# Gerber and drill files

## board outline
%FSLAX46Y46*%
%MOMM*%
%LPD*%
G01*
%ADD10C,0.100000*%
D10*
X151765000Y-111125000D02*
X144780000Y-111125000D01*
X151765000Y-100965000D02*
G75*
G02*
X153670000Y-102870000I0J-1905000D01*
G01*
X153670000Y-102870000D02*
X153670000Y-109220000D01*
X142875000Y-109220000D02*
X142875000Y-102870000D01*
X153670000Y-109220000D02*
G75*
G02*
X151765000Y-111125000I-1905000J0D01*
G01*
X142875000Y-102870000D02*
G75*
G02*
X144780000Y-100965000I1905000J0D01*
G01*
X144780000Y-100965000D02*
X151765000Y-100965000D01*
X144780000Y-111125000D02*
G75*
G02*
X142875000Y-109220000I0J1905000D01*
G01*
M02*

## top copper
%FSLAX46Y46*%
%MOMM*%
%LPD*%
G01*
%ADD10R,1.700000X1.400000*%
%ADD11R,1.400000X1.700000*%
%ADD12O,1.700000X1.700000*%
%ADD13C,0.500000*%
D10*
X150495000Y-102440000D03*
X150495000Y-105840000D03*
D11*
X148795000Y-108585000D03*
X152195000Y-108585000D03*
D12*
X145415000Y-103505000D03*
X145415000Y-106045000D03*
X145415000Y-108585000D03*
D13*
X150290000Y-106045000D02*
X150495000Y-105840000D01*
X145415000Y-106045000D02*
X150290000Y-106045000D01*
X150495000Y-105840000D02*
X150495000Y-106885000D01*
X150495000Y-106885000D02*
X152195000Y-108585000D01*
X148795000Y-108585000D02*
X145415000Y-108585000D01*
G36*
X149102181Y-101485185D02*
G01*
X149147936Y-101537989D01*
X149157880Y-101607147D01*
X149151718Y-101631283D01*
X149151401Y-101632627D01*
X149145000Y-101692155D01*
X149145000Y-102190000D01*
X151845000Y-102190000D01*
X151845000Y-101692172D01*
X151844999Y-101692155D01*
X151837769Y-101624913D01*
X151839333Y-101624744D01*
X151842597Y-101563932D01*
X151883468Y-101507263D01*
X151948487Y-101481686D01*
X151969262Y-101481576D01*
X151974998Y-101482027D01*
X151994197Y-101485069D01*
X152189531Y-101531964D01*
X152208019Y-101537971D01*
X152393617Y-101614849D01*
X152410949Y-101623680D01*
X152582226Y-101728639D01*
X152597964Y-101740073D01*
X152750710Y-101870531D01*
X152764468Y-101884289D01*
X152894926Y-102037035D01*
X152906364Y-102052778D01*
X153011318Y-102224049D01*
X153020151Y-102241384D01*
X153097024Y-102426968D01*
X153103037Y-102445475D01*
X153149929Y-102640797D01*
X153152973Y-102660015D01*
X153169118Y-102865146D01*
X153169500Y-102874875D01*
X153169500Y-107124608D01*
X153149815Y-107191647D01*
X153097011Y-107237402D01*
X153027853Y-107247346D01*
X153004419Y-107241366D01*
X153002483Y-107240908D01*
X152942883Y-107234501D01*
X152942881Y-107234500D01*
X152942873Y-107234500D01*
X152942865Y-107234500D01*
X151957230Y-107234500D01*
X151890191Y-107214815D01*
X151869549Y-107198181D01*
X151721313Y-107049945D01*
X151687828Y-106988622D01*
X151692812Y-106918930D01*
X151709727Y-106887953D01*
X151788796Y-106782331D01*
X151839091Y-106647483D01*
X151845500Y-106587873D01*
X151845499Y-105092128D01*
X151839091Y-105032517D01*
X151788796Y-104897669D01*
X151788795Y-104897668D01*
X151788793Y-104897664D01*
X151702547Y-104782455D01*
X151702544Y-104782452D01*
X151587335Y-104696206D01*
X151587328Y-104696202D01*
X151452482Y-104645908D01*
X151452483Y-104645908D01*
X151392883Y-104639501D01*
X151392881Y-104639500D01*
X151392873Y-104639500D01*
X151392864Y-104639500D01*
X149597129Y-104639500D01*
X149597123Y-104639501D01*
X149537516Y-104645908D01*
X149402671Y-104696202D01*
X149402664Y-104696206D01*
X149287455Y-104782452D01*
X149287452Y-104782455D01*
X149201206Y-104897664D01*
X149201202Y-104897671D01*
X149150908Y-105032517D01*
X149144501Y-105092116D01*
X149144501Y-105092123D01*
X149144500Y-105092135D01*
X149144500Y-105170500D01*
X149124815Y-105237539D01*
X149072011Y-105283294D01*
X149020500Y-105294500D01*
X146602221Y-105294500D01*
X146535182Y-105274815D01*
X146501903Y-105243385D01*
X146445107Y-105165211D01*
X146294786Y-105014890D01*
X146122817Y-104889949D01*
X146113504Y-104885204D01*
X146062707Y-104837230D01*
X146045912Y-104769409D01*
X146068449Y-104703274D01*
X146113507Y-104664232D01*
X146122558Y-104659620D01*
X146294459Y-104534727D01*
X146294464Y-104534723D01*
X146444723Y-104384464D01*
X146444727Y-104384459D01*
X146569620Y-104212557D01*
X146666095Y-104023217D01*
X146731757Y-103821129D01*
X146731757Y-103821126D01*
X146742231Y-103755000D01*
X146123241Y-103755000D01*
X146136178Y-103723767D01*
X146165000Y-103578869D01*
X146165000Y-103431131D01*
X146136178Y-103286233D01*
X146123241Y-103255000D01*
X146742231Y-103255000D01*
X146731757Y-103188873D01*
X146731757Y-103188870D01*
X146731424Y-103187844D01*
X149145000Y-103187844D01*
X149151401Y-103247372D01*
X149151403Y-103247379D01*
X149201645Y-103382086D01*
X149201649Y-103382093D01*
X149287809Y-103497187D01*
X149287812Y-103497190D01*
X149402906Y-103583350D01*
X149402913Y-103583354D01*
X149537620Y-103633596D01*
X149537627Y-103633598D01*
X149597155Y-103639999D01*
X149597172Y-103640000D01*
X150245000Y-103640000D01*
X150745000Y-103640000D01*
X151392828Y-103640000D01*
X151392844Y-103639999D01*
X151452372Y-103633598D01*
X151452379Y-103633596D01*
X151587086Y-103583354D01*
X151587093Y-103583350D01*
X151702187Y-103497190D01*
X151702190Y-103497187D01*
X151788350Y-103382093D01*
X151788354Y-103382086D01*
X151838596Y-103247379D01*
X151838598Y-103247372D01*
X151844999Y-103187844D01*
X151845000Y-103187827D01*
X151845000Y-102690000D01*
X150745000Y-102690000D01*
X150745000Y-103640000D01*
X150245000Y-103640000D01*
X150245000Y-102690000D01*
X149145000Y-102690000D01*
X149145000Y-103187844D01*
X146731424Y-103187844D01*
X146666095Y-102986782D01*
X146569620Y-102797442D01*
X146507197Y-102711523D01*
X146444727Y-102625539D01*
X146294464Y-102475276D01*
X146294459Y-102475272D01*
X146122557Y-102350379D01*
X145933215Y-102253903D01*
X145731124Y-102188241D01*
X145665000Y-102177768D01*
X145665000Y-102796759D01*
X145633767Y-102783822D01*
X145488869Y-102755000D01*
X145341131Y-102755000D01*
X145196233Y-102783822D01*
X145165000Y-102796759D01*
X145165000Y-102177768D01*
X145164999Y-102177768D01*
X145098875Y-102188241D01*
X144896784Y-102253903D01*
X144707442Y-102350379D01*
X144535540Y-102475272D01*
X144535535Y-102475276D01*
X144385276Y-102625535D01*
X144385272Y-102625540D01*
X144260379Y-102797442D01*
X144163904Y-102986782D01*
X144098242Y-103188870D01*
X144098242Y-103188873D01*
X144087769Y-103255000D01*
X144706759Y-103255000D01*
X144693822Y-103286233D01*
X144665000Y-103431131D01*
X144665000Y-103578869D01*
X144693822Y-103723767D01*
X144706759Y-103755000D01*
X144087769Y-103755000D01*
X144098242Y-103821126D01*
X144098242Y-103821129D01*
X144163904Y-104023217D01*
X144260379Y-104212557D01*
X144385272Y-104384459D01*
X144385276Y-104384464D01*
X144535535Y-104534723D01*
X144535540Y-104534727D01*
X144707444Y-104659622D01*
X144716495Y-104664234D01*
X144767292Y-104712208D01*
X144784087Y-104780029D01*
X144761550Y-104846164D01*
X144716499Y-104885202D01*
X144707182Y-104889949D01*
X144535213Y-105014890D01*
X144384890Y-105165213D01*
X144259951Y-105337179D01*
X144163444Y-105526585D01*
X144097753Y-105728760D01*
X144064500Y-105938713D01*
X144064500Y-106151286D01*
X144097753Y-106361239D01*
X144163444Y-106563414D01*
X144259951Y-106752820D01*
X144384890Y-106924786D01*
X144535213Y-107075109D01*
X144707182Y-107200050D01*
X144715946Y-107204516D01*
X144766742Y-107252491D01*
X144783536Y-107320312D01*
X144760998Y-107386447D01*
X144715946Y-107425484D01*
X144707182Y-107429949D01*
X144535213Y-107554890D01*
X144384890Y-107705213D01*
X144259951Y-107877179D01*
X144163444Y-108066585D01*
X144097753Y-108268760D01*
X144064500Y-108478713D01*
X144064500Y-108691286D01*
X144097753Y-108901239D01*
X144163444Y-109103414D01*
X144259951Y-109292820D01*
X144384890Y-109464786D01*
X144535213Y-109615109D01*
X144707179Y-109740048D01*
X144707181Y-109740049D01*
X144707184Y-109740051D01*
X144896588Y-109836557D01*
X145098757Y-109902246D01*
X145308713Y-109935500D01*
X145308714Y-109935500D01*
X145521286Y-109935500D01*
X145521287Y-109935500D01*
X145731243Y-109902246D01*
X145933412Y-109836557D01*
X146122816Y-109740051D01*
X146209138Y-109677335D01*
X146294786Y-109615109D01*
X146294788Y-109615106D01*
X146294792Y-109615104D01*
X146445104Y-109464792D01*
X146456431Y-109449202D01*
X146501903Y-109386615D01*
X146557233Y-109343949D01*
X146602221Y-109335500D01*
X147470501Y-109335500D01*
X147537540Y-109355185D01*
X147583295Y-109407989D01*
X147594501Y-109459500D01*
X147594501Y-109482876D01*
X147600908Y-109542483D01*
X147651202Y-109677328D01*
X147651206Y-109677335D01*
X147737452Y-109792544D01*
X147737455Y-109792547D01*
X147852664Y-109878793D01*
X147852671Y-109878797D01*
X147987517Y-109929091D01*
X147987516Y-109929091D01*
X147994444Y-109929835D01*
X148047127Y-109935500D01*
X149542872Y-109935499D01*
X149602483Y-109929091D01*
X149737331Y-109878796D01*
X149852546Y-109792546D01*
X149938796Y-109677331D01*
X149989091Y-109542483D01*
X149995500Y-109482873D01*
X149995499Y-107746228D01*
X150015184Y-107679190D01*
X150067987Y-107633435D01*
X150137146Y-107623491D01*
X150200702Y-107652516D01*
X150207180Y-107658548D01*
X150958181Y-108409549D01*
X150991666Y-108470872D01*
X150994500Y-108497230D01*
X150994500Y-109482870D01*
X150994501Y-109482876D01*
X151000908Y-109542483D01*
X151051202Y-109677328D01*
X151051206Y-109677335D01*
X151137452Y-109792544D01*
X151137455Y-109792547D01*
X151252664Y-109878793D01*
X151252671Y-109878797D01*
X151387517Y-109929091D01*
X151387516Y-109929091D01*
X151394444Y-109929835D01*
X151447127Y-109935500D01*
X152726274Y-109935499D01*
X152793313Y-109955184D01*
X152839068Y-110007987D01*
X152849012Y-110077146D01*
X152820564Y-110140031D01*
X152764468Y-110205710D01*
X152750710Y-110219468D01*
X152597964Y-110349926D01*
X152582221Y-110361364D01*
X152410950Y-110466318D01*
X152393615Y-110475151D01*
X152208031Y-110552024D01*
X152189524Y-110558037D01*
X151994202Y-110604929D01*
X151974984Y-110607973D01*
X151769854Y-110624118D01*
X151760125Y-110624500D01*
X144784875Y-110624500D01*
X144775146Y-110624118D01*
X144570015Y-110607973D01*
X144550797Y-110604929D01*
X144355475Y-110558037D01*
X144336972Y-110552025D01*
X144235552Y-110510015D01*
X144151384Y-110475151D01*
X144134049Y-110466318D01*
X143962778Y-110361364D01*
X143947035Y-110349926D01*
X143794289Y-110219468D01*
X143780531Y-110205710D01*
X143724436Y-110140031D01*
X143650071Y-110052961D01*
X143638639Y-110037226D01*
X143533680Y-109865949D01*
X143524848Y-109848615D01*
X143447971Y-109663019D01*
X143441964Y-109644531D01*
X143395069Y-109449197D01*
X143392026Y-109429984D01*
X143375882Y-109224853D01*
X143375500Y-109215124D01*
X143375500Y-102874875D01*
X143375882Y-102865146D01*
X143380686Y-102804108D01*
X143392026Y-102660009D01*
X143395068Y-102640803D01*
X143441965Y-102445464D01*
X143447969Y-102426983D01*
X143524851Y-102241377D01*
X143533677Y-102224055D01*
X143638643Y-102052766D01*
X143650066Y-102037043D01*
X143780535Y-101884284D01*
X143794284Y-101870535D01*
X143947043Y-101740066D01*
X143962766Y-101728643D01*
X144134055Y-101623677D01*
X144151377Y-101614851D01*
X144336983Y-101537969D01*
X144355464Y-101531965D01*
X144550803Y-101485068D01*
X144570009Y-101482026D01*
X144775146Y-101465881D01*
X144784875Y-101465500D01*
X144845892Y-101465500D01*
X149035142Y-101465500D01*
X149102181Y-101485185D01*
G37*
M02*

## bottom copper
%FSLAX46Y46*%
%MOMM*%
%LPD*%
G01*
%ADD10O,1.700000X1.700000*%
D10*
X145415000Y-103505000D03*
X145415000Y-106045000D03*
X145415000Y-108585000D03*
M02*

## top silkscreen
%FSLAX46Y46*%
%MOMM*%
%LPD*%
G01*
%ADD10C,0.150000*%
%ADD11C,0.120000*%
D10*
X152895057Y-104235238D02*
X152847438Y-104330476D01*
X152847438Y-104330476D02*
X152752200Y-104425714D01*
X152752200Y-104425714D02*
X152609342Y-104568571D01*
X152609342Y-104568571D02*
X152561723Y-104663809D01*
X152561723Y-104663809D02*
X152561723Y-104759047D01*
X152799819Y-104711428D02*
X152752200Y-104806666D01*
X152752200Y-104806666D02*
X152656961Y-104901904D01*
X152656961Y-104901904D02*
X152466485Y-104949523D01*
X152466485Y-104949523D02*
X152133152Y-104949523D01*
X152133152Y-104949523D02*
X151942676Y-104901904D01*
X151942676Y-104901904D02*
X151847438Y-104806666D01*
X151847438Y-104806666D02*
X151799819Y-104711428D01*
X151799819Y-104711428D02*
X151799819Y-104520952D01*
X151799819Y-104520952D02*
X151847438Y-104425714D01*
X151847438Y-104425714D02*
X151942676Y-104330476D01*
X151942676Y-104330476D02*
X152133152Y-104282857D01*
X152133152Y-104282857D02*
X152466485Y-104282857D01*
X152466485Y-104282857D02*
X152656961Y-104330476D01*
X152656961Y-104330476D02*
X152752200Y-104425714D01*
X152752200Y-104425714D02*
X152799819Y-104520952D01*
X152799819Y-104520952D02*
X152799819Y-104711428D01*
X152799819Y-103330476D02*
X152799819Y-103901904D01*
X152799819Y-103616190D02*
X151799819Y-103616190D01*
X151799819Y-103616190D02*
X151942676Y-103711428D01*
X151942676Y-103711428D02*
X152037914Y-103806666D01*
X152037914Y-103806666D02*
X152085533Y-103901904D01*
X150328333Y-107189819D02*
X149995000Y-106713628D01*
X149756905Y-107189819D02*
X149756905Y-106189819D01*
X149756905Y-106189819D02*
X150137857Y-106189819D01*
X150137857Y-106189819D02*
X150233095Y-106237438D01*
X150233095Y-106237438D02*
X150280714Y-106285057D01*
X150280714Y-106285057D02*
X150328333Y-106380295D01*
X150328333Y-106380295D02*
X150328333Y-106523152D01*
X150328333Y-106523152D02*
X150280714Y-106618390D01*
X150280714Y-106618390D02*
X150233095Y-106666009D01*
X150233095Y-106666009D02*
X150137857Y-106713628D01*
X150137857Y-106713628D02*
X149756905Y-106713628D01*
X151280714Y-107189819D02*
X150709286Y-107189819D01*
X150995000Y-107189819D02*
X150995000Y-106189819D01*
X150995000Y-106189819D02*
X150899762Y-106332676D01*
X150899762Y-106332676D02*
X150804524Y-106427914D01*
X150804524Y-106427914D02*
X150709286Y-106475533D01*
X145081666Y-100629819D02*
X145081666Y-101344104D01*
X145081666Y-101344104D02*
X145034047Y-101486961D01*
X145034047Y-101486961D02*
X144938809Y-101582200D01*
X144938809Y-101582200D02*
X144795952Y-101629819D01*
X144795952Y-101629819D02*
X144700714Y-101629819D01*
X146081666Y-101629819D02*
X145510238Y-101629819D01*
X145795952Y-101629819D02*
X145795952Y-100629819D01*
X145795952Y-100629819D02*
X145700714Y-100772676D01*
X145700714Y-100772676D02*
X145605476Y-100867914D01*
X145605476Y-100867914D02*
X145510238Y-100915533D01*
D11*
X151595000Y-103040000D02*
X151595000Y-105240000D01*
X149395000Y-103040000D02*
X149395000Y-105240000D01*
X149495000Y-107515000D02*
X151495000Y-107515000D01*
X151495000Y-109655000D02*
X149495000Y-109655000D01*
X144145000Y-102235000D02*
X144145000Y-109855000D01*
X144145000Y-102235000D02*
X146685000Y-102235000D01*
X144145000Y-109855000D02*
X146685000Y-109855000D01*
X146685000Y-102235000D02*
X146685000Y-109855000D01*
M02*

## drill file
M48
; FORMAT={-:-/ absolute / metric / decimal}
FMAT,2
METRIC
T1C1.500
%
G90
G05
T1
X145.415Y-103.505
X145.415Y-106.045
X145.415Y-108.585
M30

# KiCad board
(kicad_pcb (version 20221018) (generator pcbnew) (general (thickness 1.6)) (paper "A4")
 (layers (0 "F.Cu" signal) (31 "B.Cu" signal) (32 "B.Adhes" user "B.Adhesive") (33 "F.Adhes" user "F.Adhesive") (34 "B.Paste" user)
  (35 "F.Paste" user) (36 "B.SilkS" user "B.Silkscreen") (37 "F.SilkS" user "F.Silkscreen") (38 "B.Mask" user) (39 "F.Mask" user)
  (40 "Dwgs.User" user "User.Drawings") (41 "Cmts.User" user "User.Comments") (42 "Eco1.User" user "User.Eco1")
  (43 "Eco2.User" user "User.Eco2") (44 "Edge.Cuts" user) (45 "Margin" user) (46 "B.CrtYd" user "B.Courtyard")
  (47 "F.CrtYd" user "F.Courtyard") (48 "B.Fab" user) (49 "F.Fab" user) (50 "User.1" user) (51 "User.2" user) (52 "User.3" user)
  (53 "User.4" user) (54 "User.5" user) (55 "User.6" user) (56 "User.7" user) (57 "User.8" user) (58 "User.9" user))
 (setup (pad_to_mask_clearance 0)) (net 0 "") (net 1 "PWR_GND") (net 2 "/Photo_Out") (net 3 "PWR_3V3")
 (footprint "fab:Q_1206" (layer "F.Cu") (at 150.495 104.14 -90)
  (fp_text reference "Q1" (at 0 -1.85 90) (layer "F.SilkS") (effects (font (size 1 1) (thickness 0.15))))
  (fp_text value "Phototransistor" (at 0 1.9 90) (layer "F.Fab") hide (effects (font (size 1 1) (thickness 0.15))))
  (fp_line (start -1.1 -1.1) (end 1.1 -1.1) (stroke (width 0.12) (type default)) (layer "F.SilkS"))
  (fp_line (start -1.1 1.1) (end 1.1 1.1) (stroke (width 0.12) (type default)) (layer "F.SilkS"))
  (pad "1" smd rect (at -1.7 0 270) (size 1.4 1.7) (layers "F.Cu" "F.Paste" "F.Mask") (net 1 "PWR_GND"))
  (pad "2" smd rect (at 1.7 0 270) (size 1.4 1.7) (layers "F.Cu" "F.Paste" "F.Mask") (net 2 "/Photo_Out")))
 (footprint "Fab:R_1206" (layer "F.Cu") (at 150.495 108.585)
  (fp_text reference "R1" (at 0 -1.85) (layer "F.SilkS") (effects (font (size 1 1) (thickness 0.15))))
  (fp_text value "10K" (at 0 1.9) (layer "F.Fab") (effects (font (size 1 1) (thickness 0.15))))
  (fp_line (start -1 -1.07) (end 1 -1.07) (stroke (width 0.12) (type solid)) (layer "F.SilkS"))
  (fp_line (start 1 1.07) (end -1 1.07) (stroke (width 0.12) (type solid)) (layer "F.SilkS"))
  (pad "1" smd rect (at -1.7 0) (size 1.4 1.7) (layers "F.Cu" "F.Paste" "F.Mask") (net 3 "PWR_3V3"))
  (pad "2" smd rect (at 1.7 0) (size 1.4 1.7) (layers "F.Cu" "F.Paste" "F.Mask") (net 2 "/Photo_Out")))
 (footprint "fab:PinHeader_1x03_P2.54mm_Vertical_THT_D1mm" (layer "F.Cu") (at 145.415 103.505)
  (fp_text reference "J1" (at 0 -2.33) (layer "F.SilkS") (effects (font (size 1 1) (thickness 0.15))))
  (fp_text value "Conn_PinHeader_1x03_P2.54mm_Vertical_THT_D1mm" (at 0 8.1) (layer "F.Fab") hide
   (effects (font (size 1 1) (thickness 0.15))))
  (fp_line (start -1.27 -1.27) (end -1.27 6.35) (stroke (width 0.12) (type solid)) (layer "F.SilkS"))
  (fp_line (start -1.27 -1.27) (end 1.27 -1.27) (stroke (width 0.12) (type solid)) (layer "F.SilkS"))
  (fp_line (start -1.27 6.35) (end 1.27 6.35) (stroke (width 0.12) (type solid)) (layer "F.SilkS"))
  (fp_line (start 1.27 -1.27) (end 1.27 6.35) (stroke (width 0.12) (type solid)) (layer "F.SilkS"))
  (pad "1" thru_hole oval (at 0 0) (size 1.7 1.7) (drill 1.5) (layers "*.Cu" "*.Mask") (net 1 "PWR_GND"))
  (pad "2" thru_hole oval (at 0 2.54) (size 1.7 1.7) (drill 1.5) (layers "*.Cu" "*.Mask") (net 2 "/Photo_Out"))
  (pad "3" thru_hole oval (at 0 5.08) (size 1.7 1.7) (drill 1.5) (layers "*.Cu" "*.Mask") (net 3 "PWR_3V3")))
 (gr_line (start 151.765 111.125) (end 144.78 111.125) (stroke (width 0.1) (type default)) (layer "Edge.Cuts"))
 (gr_arc (start 151.765 100.965) (mid 153.112038 101.522962) (end 153.67 102.87) (stroke (width 0.1) (type default)) (layer "Edge.Cuts"))
 (gr_line (start 153.67 102.87) (end 153.67 109.22) (stroke (width 0.1) (type default)) (layer "Edge.Cuts"))
 (gr_line (start 142.875 109.22) (end 142.875 102.87) (stroke (width 0.1) (type default)) (layer "Edge.Cuts"))
 (gr_arc (start 153.67 109.22) (mid 153.112038 110.567038) (end 151.765 111.125) (stroke (width 0.1) (type default)) (layer "Edge.Cuts"))
 (gr_arc (start 142.875 102.87) (mid 143.432962 101.522962) (end 144.78 100.965) (stroke (width 0.1) (type default)) (layer "Edge.Cuts"))
 (gr_line (start 144.78 100.965) (end 151.765 100.965) (stroke (width 0.1) (type default)) (layer "Edge.Cuts"))
 (gr_arc (start 144.78 111.125) (mid 143.432962 110.567038) (end 142.875 109.22) (stroke (width 0.1) (type default)) (layer "Edge.Cuts"))
 (segment (start 150.29 106.045) (end 150.495 105.84) (width 0.5) (layer "F.Cu") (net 2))
 (segment (start 145.415 106.045) (end 150.29 106.045) (width 0.5) (layer "F.Cu") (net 2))
 (segment (start 150.495 105.84) (end 150.495 106.885) (width 0.5) (layer "F.Cu") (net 2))
 (segment (start 150.495 106.885) (end 152.195 108.585) (width 0.5) (layer "F.Cu") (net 2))
 (segment (start 148.795 108.585) (end 145.415 108.585) (width 0.5) (layer "F.Cu") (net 3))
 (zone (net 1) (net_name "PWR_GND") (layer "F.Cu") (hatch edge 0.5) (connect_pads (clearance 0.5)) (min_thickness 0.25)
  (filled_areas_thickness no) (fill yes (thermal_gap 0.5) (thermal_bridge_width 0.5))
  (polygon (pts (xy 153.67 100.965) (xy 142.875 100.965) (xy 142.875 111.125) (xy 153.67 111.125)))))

